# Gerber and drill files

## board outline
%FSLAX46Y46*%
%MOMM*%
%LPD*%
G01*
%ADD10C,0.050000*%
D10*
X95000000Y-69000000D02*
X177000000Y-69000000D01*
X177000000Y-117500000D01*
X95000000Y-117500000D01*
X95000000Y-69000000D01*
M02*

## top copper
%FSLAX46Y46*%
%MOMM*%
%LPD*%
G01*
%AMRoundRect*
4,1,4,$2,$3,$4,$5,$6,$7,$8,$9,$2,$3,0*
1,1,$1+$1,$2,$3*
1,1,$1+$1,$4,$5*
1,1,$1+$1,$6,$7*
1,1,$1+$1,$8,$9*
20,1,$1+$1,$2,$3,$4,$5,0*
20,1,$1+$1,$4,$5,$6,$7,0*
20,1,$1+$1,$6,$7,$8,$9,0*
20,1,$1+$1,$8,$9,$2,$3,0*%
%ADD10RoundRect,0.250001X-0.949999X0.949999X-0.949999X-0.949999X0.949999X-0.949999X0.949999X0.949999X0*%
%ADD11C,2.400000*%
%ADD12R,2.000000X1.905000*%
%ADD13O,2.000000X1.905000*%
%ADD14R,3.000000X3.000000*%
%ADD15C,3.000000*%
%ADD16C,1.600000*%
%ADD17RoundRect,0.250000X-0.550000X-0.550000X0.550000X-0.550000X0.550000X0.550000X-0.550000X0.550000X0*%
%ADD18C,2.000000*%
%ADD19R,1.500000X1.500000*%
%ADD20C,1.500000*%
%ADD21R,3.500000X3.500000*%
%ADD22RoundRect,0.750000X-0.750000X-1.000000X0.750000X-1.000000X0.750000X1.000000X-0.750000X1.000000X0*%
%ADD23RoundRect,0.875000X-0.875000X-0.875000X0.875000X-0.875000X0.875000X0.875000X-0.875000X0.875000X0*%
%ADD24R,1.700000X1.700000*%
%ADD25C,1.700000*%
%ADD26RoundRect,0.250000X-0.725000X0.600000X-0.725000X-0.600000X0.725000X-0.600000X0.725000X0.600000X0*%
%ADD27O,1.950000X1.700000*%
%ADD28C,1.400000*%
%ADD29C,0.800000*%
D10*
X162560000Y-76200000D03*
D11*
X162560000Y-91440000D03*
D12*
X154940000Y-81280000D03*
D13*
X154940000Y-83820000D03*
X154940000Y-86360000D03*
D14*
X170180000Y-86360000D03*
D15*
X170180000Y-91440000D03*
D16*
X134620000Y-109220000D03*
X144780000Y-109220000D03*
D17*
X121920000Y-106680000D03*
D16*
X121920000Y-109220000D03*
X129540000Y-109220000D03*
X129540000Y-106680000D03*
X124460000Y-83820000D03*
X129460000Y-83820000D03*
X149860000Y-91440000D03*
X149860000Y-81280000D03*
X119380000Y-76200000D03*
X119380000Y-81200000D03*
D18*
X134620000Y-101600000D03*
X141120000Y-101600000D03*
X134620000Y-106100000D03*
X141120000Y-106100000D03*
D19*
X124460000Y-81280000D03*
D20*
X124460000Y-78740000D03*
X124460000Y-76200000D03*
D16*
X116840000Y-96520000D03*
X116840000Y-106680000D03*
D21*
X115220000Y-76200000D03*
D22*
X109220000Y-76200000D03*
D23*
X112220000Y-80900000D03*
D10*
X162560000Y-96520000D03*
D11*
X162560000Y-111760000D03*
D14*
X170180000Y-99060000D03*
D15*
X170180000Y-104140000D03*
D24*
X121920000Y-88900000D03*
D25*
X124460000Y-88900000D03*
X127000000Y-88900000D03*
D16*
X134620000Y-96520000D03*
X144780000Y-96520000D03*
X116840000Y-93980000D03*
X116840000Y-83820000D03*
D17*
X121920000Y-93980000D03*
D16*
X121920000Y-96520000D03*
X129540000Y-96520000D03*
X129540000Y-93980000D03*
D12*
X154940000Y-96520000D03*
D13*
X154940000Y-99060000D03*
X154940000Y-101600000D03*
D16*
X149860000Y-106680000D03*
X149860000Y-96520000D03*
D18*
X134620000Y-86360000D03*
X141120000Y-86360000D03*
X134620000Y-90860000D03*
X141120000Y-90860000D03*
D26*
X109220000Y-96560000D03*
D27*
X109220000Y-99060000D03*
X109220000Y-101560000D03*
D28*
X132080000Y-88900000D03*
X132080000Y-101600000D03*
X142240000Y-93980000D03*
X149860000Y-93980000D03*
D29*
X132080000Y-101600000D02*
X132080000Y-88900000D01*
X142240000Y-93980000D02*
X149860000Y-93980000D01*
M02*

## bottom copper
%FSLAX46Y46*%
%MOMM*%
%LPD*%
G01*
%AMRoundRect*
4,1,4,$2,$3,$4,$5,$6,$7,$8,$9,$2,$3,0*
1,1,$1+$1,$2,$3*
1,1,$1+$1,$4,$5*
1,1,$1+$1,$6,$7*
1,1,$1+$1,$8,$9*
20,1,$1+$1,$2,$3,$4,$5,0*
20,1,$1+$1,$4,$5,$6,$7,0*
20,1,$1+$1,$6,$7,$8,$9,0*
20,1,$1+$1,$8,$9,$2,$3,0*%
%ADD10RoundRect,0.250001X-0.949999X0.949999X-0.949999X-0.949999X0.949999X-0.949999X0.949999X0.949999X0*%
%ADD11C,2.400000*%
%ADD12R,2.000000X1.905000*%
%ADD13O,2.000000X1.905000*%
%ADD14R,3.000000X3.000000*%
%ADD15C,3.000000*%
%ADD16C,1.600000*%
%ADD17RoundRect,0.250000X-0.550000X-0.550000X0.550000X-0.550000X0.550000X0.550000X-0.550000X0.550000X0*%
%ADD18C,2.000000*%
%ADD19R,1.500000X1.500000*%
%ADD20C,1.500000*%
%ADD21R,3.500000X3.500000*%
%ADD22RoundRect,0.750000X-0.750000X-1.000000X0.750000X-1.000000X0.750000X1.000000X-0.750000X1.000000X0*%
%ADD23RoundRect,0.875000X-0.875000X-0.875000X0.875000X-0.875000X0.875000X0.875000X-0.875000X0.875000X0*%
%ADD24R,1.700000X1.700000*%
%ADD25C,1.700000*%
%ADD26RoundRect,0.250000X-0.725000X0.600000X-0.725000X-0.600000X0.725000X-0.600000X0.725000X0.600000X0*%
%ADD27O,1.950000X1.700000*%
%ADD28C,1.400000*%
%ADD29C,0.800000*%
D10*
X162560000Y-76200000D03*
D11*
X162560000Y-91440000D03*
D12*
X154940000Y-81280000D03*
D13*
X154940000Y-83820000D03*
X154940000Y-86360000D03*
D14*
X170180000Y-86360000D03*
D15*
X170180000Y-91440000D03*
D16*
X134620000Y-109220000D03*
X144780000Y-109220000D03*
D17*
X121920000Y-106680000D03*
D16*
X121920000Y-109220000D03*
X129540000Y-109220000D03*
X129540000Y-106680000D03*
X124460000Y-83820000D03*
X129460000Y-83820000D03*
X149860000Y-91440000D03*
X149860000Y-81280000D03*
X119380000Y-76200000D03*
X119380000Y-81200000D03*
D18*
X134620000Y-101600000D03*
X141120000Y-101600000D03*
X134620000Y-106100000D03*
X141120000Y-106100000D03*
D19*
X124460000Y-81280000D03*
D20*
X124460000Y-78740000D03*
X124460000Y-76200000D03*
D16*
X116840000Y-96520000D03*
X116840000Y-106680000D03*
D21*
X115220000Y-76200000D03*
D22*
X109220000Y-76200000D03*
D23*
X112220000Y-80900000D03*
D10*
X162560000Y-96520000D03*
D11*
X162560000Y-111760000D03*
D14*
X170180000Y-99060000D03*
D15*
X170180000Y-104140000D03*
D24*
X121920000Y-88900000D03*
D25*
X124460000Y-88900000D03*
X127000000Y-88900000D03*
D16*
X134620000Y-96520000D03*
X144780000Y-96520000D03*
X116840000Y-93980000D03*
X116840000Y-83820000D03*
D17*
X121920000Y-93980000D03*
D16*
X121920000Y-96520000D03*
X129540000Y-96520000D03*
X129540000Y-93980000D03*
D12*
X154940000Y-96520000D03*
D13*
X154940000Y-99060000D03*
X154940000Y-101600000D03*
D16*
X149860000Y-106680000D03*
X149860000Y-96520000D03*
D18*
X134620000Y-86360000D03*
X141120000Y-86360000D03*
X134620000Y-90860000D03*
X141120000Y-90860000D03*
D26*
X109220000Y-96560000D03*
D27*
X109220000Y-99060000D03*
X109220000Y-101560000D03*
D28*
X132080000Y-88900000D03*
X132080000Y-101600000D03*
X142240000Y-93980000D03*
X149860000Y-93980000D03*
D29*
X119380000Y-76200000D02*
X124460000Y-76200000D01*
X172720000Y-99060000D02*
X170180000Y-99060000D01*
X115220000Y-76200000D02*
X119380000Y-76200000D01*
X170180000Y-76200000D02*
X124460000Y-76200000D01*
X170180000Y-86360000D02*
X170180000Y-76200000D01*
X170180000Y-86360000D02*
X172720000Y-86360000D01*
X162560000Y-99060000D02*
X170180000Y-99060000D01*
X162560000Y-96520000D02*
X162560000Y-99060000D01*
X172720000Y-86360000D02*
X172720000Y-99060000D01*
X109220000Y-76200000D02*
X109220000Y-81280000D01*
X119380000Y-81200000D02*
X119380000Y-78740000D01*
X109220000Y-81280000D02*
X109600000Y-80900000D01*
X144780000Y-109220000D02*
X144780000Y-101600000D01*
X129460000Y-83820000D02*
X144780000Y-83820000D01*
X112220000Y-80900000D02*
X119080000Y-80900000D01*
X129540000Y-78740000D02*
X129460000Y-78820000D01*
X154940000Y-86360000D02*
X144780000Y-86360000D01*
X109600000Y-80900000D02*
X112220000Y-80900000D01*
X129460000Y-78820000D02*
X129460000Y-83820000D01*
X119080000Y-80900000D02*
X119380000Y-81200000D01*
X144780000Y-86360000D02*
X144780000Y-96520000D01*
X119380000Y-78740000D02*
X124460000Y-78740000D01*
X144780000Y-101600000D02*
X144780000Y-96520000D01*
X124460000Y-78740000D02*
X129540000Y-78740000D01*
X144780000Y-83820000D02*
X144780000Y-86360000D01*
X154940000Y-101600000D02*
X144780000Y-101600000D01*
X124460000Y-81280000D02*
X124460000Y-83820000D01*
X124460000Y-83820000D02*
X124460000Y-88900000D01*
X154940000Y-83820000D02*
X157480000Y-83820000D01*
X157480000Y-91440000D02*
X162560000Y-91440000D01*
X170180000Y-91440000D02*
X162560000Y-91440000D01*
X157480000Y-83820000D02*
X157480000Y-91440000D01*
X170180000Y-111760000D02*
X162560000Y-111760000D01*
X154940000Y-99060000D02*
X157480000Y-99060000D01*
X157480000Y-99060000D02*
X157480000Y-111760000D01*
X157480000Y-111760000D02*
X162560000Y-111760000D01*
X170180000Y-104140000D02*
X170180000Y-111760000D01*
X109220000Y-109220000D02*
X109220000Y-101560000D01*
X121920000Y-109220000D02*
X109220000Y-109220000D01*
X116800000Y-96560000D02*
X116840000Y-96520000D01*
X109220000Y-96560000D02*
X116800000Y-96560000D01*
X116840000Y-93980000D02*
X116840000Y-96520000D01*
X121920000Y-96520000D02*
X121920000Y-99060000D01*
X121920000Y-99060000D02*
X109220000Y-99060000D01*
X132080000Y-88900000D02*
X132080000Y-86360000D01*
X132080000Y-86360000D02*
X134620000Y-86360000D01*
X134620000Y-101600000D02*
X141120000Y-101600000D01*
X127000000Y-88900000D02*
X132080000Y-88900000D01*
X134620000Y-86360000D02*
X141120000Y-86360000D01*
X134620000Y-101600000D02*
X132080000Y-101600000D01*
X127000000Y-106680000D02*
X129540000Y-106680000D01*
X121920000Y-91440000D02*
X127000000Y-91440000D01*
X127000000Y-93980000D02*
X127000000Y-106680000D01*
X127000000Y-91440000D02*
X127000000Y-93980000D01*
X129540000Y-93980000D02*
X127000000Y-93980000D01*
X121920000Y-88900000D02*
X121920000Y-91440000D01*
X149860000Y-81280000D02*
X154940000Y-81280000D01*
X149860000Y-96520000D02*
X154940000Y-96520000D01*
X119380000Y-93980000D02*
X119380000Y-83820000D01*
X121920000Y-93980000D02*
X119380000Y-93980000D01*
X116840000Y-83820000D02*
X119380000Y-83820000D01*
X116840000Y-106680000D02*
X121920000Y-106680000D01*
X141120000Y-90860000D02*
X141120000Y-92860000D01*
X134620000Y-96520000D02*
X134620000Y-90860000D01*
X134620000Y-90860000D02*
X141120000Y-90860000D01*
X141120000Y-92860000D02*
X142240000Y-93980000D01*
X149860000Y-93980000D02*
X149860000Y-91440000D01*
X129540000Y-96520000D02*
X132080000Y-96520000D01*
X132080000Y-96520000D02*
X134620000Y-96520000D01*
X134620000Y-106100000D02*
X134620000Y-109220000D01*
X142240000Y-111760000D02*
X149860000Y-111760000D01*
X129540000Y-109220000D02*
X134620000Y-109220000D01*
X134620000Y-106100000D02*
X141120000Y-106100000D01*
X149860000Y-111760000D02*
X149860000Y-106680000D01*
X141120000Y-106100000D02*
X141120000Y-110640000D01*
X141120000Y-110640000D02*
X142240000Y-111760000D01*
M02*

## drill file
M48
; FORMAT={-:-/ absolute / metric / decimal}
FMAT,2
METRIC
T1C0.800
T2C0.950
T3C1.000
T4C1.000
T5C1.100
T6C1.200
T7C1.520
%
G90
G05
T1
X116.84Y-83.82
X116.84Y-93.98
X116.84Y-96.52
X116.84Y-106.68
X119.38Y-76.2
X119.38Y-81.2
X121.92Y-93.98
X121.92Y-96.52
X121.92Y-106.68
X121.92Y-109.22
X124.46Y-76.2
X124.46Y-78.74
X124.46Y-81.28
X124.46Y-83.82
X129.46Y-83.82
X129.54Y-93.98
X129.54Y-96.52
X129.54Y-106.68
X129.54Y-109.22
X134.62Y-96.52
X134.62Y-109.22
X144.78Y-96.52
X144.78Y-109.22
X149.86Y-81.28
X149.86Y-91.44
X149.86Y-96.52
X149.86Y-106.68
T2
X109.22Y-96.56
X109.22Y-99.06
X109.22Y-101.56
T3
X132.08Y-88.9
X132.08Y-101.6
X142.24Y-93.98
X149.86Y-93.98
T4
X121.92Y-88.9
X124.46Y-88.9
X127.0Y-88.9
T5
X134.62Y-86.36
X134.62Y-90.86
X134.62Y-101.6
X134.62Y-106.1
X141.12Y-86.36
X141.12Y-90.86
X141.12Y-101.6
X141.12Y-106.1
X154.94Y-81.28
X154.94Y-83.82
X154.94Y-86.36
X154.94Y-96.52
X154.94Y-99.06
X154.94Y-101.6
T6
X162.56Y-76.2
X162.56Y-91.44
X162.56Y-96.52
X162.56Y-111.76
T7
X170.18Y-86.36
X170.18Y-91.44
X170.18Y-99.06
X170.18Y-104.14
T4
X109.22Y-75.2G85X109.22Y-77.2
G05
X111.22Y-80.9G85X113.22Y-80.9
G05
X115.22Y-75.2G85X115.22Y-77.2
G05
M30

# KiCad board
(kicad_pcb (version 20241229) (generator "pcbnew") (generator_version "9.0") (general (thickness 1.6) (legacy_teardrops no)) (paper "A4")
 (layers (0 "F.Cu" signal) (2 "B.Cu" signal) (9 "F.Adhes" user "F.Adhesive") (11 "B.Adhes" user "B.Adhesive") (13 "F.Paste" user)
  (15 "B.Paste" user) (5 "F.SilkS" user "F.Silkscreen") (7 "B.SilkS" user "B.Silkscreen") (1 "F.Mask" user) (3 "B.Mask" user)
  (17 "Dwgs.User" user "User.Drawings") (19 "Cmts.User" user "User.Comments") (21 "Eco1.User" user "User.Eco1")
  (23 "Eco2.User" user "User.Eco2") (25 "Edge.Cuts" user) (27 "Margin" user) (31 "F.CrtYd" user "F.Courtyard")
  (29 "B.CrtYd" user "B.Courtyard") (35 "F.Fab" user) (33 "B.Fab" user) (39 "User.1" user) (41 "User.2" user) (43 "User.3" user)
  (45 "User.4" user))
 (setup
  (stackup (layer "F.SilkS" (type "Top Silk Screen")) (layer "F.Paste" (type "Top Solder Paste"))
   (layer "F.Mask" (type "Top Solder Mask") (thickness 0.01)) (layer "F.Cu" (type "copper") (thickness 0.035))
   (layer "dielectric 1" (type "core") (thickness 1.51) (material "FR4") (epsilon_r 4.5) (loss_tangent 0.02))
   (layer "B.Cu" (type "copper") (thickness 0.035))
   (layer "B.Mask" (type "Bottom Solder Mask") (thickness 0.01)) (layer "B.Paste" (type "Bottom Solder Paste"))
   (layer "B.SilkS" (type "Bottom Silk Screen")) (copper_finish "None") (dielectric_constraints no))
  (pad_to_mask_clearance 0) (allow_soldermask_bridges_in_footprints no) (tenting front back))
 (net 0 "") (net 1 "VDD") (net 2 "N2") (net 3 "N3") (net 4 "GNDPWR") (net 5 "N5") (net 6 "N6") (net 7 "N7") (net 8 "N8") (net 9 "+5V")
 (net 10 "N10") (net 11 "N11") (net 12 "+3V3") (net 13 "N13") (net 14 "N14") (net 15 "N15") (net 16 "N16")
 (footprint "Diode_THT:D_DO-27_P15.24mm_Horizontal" (layer "F.Cu") (at 162.56 76.2 -90)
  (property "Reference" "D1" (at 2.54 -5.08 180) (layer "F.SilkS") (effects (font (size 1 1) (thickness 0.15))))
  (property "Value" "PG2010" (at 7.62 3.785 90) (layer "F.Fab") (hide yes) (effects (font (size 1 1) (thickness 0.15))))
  (pad "1" thru_hole roundrect (at 0 0 270) (size 2.4 2.4) (drill 1.2) (layers "*.Cu" "*.Mask") (remove_unused_layers no)
   (roundrect_rratio 0.104167) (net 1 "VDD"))
  (pad "2" thru_hole circle (at 15.24 0 270) (size 2.4 2.4) (drill 1.2) (layers "*.Cu" "*.Mask") (remove_unused_layers no) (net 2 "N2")))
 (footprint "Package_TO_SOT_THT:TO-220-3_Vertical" (layer "F.Cu") (at 154.94 81.28 -90)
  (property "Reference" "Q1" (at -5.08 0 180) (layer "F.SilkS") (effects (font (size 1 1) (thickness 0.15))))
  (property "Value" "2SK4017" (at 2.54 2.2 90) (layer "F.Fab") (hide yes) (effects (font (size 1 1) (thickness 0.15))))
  (pad "1" thru_hole rect (at 0 0 270) (size 1.905 2) (drill 1.1) (layers "*.Cu" "*.Mask") (remove_unused_layers no) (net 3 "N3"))
  (pad "2" thru_hole oval (at 2.54 0 270) (size 1.905 2) (drill 1.1) (layers "*.Cu" "*.Mask") (remove_unused_layers no) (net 2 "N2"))
  (pad "3" thru_hole oval (at 5.08 0 270) (size 1.905 2) (drill 1.1) (layers "*.Cu" "*.Mask") (remove_unused_layers no) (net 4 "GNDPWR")))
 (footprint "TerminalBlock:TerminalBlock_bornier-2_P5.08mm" (layer "F.Cu") (at 170.18 86.36 -90)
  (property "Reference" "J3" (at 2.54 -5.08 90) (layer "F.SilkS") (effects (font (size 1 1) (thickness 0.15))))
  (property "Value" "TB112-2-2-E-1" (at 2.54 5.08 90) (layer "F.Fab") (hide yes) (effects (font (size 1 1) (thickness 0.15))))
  (pad "1" thru_hole rect (at 0 0 270) (size 3 3) (drill 1.52) (layers "*.Cu" "*.Mask") (remove_unused_layers no) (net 1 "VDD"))
  (pad "2" thru_hole circle (at 5.08 0 270) (size 3 3) (drill 1.52) (layers "*.Cu" "*.Mask") (remove_unused_layers no) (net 2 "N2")))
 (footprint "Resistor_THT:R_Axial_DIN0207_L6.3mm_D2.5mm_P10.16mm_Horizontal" (layer "F.Cu") (at 134.62 109.22)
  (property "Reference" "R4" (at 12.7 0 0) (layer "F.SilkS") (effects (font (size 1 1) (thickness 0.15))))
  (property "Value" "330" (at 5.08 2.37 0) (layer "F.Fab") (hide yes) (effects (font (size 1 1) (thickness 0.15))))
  (pad "1" thru_hole circle (at 0 0) (size 1.6 1.6) (drill 0.8) (layers "*.Cu" "*.Mask") (remove_unused_layers no) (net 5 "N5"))
  (pad "2" thru_hole circle (at 10.16 0) (size 1.6 1.6) (drill 0.8) (layers "*.Cu" "*.Mask") (remove_unused_layers no) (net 4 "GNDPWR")))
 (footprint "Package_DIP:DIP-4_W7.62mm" (layer "F.Cu") (at 121.92 106.68)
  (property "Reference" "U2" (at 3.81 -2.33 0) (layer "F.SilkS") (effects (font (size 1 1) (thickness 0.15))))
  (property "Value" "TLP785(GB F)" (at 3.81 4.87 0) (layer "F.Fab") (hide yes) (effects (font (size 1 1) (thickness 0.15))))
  (pad "1" thru_hole roundrect (at 0 0) (size 1.6 1.6) (drill 0.8) (layers "*.Cu" "*.Mask") (remove_unused_layers no)
   (roundrect_rratio 0.15625) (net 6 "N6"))
  (pad "2" thru_hole circle (at 0 2.54) (size 1.6 1.6) (drill 0.8) (layers "*.Cu" "*.Mask") (remove_unused_layers no) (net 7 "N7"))
  (pad "3" thru_hole circle (at 7.62 2.54) (size 1.6 1.6) (drill 0.8) (layers "*.Cu" "*.Mask") (remove_unused_layers no) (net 5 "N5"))
  (pad "4" thru_hole circle (at 7.62 0) (size 1.6 1.6) (drill 0.8) (layers "*.Cu" "*.Mask") (remove_unused_layers no) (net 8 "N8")))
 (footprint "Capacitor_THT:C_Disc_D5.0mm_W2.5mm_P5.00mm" (layer "F.Cu") (at 124.46 83.82)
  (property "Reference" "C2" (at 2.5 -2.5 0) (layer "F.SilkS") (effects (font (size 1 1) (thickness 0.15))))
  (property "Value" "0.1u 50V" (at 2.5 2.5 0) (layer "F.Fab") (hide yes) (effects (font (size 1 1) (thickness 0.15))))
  (pad "1" thru_hole circle (at 0 0) (size 1.6 1.6) (drill 0.8) (layers "*.Cu" "*.Mask") (remove_unused_layers no) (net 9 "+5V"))
  (pad "2" thru_hole circle (at 5 0) (size 1.6 1.6) (drill 0.8) (layers "*.Cu" "*.Mask") (remove_unused_layers no) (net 4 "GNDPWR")))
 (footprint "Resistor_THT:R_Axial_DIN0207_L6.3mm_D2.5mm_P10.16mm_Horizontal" (layer "F.Cu") (at 149.86 91.44 90)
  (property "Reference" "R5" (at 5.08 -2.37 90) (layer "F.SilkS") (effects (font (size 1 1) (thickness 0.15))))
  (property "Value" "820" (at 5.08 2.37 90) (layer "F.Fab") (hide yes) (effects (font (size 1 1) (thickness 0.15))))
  (pad "1" thru_hole circle (at 0 0 90) (size 1.6 1.6) (drill 0.8) (layers "*.Cu" "*.Mask") (remove_unused_layers no) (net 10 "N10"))
  (pad "2" thru_hole circle (at 10.16 0 90) (size 1.6 1.6) (drill 0.8) (layers "*.Cu" "*.Mask") (remove_unused_layers no) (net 3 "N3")))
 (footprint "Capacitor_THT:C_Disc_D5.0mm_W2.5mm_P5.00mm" (layer "F.Cu") (at 119.38 76.2 -90)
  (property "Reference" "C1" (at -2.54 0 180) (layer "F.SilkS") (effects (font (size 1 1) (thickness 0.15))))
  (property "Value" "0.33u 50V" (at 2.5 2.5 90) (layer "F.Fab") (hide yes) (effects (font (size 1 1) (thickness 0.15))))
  (pad "1" thru_hole circle (at 0 0 270) (size 1.6 1.6) (drill 0.8) (layers "*.Cu" "*.Mask") (remove_unused_layers no) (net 1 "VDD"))
  (pad "2" thru_hole circle (at 5 0 270) (size 1.6 1.6) (drill 0.8) (layers "*.Cu" "*.Mask") (remove_unused_layers no) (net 4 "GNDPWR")))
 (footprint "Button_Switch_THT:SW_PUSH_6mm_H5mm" (layer "F.Cu") (at 134.62 101.6)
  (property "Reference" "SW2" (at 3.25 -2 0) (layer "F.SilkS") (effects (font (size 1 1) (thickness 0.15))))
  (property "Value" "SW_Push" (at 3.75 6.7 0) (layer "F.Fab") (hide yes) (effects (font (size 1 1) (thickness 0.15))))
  (pad "1" thru_hole circle (at 0 0 90) (size 2 2) (drill 1.1) (layers "*.Cu" "*.Mask") (remove_unused_layers no) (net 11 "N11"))
  (pad "1" thru_hole circle (at 6.5 0 90) (size 2 2) (drill 1.1) (layers "*.Cu" "*.Mask") (remove_unused_layers no) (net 11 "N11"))
  (pad "2" thru_hole circle (at 0 4.5 90) (size 2 2) (drill 1.1) (layers "*.Cu" "*.Mask") (remove_unused_layers no) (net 5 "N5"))
  (pad "2" thru_hole circle (at 6.5 4.5 90) (size 2 2) (drill 1.1) (layers "*.Cu" "*.Mask") (remove_unused_layers no) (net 5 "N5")))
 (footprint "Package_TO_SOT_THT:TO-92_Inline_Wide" (layer "F.Cu") (at 124.46 81.28 90)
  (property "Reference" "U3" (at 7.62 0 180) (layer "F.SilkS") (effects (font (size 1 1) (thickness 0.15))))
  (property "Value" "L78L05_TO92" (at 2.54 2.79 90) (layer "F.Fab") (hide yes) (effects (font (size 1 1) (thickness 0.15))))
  (pad "1" thru_hole rect (at 0 0 90) (size 1.5 1.5) (drill 0.8) (layers "*.Cu" "*.Mask") (remove_unused_layers no) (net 9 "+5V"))
  (pad "2" thru_hole circle (at 2.54 0 90) (size 1.5 1.5) (drill 0.8) (layers "*.Cu" "*.Mask") (remove_unused_layers no) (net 4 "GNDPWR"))
  (pad "3" thru_hole circle (at 5.08 0 90) (size 1.5 1.5) (drill 0.8) (layers "*.Cu" "*.Mask") (remove_unused_layers no) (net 1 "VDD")))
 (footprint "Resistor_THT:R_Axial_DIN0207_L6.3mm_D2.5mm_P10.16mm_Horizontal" (layer "F.Cu") (at 116.84 96.52 -90)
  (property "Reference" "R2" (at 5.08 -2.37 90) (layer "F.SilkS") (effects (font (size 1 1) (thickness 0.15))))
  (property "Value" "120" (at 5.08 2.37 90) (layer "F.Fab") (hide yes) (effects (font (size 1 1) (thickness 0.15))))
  (pad "1" thru_hole circle (at 0 0 270) (size 1.6 1.6) (drill 0.8) (layers "*.Cu" "*.Mask") (remove_unused_layers no) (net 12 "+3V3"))
  (pad "2" thru_hole circle (at 10.16 0 270) (size 1.6 1.6) (drill 0.8) (layers "*.Cu" "*.Mask") (remove_unused_layers no) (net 6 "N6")))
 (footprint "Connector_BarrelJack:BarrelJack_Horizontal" (layer "F.Cu") (at 115.22 76.2)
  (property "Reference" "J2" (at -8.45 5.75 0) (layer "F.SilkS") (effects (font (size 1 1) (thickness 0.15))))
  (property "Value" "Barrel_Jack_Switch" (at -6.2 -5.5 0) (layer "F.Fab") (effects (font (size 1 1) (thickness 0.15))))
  (pad "1" thru_hole rect (at 0 0) (size 3.5 3.5) (drill oval 1 3) (layers "*.Cu" "*.Mask") (remove_unused_layers no) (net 1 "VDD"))
  (pad "2" thru_hole roundrect (at -6 0) (size 3 3.5) (drill oval 1 3) (layers "*.Cu" "*.Mask") (remove_unused_layers no)
   (roundrect_rratio 0.25) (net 4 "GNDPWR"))
  (pad "3" thru_hole roundrect (at -3 4.7) (size 3.5 3.5) (drill oval 3 1) (layers "*.Cu" "*.Mask") (remove_unused_layers no)
   (roundrect_rratio 0.25) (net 4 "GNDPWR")))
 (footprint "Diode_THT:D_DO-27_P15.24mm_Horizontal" (layer "F.Cu") (at 162.56 96.52 -90)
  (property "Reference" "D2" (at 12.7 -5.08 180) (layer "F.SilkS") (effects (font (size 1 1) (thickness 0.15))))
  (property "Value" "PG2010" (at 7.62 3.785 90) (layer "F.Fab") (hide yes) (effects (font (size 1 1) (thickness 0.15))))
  (pad "1" thru_hole roundrect (at 0 0 270) (size 2.4 2.4) (drill 1.2) (layers "*.Cu" "*.Mask") (remove_unused_layers no)
   (roundrect_rratio 0.104167) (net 1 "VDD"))
  (pad "2" thru_hole circle (at 15.24 0 270) (size 2.4 2.4) (drill 1.2) (layers "*.Cu" "*.Mask") (remove_unused_layers no) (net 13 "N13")))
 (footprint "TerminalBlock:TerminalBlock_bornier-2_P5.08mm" (layer "F.Cu") (at 170.18 99.06 -90)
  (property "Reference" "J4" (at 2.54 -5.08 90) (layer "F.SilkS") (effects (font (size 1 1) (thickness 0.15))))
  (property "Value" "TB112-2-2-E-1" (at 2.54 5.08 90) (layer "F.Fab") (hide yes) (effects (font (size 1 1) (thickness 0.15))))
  (pad "1" thru_hole rect (at 0 0 270) (size 3 3) (drill 1.52) (layers "*.Cu" "*.Mask") (remove_unused_layers no) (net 1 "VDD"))
  (pad "2" thru_hole circle (at 5.08 0 270) (size 3 3) (drill 1.52) (layers "*.Cu" "*.Mask") (remove_unused_layers no) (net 13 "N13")))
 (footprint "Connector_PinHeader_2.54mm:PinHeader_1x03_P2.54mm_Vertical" (layer "F.Cu") (at 121.92 88.9 90)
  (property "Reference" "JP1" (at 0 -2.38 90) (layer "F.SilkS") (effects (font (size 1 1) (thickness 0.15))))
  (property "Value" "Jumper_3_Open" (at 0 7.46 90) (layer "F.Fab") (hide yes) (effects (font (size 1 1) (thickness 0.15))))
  (pad "1" thru_hole rect (at 0 0 90) (size 1.7 1.7) (drill 1) (layers "*.Cu" "*.Mask") (remove_unused_layers no) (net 8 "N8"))
  (pad "2" thru_hole circle (at 0 2.54 90) (size 1.7 1.7) (drill 1) (layers "*.Cu" "*.Mask") (remove_unused_layers no) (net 9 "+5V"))
  (pad "3" thru_hole circle (at 0 5.08 90) (size 1.7 1.7) (drill 1) (layers "*.Cu" "*.Mask") (remove_unused_layers no) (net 11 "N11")))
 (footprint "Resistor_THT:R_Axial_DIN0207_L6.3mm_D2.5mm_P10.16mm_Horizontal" (layer "F.Cu") (at 134.62 96.52)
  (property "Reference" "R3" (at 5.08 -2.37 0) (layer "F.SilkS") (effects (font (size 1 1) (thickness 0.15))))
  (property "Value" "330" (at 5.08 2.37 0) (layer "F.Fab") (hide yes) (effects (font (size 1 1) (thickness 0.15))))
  (pad "1" thru_hole circle (at 0 0) (size 1.6 1.6) (drill 0.8) (layers "*.Cu" "*.Mask") (remove_unused_layers no) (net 10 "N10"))
  (pad "2" thru_hole circle (at 10.16 0) (size 1.6 1.6) (drill 0.8) (layers "*.Cu" "*.Mask") (remove_unused_layers no) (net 4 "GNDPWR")))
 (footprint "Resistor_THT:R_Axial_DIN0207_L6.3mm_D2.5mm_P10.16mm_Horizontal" (layer "F.Cu") (at 116.84 93.98 90)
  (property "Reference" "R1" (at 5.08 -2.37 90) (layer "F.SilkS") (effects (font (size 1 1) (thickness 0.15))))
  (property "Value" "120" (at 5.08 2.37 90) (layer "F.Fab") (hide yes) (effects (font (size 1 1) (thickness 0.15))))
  (pad "1" thru_hole circle (at 0 0 90) (size 1.6 1.6) (drill 0.8) (layers "*.Cu" "*.Mask") (remove_unused_layers no) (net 12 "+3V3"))
  (pad "2" thru_hole circle (at 10.16 0 90) (size 1.6 1.6) (drill 0.8) (layers "*.Cu" "*.Mask") (remove_unused_layers no) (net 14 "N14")))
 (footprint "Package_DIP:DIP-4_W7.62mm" (layer "F.Cu") (at 121.92 93.98)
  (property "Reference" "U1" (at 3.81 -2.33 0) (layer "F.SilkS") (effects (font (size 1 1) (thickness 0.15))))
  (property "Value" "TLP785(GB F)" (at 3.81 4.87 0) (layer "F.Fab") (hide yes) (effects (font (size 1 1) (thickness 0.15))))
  (pad "1" thru_hole roundrect (at 0 0) (size 1.6 1.6) (drill 0.8) (layers "*.Cu" "*.Mask") (remove_unused_layers no)
   (roundrect_rratio 0.15625) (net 14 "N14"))
  (pad "2" thru_hole circle (at 0 2.54) (size 1.6 1.6) (drill 0.8) (layers "*.Cu" "*.Mask") (remove_unused_layers no) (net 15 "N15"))
  (pad "3" thru_hole circle (at 7.62 2.54) (size 1.6 1.6) (drill 0.8) (layers "*.Cu" "*.Mask") (remove_unused_layers no) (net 10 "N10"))
  (pad "4" thru_hole circle (at 7.62 0) (size 1.6 1.6) (drill 0.8) (layers "*.Cu" "*.Mask") (remove_unused_layers no) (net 8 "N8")))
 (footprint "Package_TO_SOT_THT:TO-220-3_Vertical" (layer "F.Cu") (at 154.94 96.52 -90)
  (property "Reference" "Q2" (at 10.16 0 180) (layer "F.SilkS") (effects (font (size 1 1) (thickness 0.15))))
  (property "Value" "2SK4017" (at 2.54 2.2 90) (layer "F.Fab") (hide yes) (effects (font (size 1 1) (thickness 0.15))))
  (pad "1" thru_hole rect (at 0 0 270) (size 1.905 2) (drill 1.1) (layers "*.Cu" "*.Mask") (remove_unused_layers no) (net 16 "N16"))
  (pad "2" thru_hole oval (at 2.54 0 270) (size 1.905 2) (drill 1.1) (layers "*.Cu" "*.Mask") (remove_unused_layers no) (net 13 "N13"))
  (pad "3" thru_hole oval (at 5.08 0 270) (size 1.905 2) (drill 1.1) (layers "*.Cu" "*.Mask") (remove_unused_layers no) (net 4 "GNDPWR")))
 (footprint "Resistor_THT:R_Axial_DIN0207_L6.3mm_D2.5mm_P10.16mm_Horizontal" (layer "F.Cu") (at 149.86 106.68 90)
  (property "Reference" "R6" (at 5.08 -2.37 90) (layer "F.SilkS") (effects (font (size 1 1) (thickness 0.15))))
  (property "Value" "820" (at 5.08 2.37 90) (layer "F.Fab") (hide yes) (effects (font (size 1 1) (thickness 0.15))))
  (pad "1" thru_hole circle (at 0 0 90) (size 1.6 1.6) (drill 0.8) (layers "*.Cu" "*.Mask") (remove_unused_layers no) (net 5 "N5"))
  (pad "2" thru_hole circle (at 10.16 0 90) (size 1.6 1.6) (drill 0.8) (layers "*.Cu" "*.Mask") (remove_unused_layers no) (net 16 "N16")))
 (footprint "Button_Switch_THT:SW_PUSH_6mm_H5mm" (layer "F.Cu") (at 134.62 86.36)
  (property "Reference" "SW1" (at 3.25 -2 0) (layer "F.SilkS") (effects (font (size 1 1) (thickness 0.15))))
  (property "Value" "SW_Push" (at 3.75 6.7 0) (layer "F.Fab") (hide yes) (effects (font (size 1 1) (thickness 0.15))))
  (pad "1" thru_hole circle (at 0 0 90) (size 2 2) (drill 1.1) (layers "*.Cu" "*.Mask") (remove_unused_layers no) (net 11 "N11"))
  (pad "1" thru_hole circle (at 6.5 0 90) (size 2 2) (drill 1.1) (layers "*.Cu" "*.Mask") (remove_unused_layers no) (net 11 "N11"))
  (pad "2" thru_hole circle (at 0 4.5 90) (size 2 2) (drill 1.1) (layers "*.Cu" "*.Mask") (remove_unused_layers no) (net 10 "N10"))
  (pad "2" thru_hole circle (at 6.5 4.5 90) (size 2 2) (drill 1.1) (layers "*.Cu" "*.Mask") (remove_unused_layers no) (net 10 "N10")))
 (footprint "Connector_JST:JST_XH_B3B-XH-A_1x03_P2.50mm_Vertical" (layer "F.Cu") (at 109.22 96.56 -90)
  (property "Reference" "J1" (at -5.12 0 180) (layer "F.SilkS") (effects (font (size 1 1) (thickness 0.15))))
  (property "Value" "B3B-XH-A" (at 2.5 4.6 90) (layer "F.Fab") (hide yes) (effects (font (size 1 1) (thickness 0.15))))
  (pad "1" thru_hole roundrect (at 0 0 270) (size 1.7 1.95) (drill 0.95) (layers "*.Cu" "*.Mask") (remove_unused_layers no)
   (roundrect_rratio 0.147059) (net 12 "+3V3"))
  (pad "2" thru_hole oval (at 2.5 0 270) (size 1.7 1.95) (drill 0.95) (layers "*.Cu" "*.Mask") (remove_unused_layers no) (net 15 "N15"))
  (pad "3" thru_hole oval (at 5 0 270) (size 1.7 1.95) (drill 0.95) (layers "*.Cu" "*.Mask") (remove_unused_layers no) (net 7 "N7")))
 (gr_rect (start 95 69) (end 177 117.5) (stroke (width 0.05) (type default)) (fill no) (layer "Edge.Cuts"))
 (segment (start 119.38 76.2) (end 124.46 76.2) (width 0.8) (layer "B.Cu") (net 1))
 (segment (start 172.72 99.06) (end 170.18 99.06) (width 0.8) (layer "B.Cu") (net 1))
 (segment (start 115.22 76.2) (end 119.38 76.2) (width 0.8) (layer "B.Cu") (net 1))
 (segment (start 170.18 76.2) (end 124.46 76.2) (width 0.8) (layer "B.Cu") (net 1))
 (segment (start 170.18 86.36) (end 170.18 76.2) (width 0.8) (layer "B.Cu") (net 1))
 (segment (start 170.18 86.36) (end 172.72 86.36) (width 0.8) (layer "B.Cu") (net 1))
 (segment (start 162.56 99.06) (end 170.18 99.06) (width 0.8) (layer "B.Cu") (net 1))
 (segment (start 162.56 96.52) (end 162.56 99.06) (width 0.8) (layer "B.Cu") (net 1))
 (segment (start 172.72 86.36) (end 172.72 99.06) (width 0.8) (layer "B.Cu") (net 1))
 (segment (start 109.22 76.2) (end 109.22 81.28) (width 0.8) (layer "B.Cu") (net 4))
 (segment (start 119.38 81.2) (end 119.38 78.74) (width 0.8) (layer "B.Cu") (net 4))
 (segment (start 109.22 81.28) (end 109.6 80.9) (width 0.8) (layer "B.Cu") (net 4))
 (segment (start 144.78 109.22) (end 144.78 101.6) (width 0.8) (layer "B.Cu") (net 4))
 (segment (start 129.46 83.82) (end 144.78 83.82) (width 0.8) (layer "B.Cu") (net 4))
 (segment (start 112.22 80.9) (end 119.08 80.9) (width 0.8) (layer "B.Cu") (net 4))
 (segment (start 129.54 78.74) (end 129.46 78.82) (width 0.8) (layer "B.Cu") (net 4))
 (segment (start 154.94 86.36) (end 144.78 86.36) (width 0.8) (layer "B.Cu") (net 4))
 (segment (start 109.6 80.9) (end 112.22 80.9) (width 0.8) (layer "B.Cu") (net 4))
 (segment (start 129.46 78.82) (end 129.46 83.82) (width 0.8) (layer "B.Cu") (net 4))
 (segment (start 119.08 80.9) (end 119.38 81.2) (width 0.8) (layer "B.Cu") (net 4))
 (segment (start 144.78 86.36) (end 144.78 96.52) (width 0.8) (layer "B.Cu") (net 4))
 (segment (start 119.38 78.74) (end 124.46 78.74) (width 0.8) (layer "B.Cu") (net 4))
 (segment (start 144.78 101.6) (end 144.78 96.52) (width 0.8) (layer "B.Cu") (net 4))
 (segment (start 124.46 78.74) (end 129.54 78.74) (width 0.8) (layer "B.Cu") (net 4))
 (segment (start 144.78 83.82) (end 144.78 86.36) (width 0.8) (layer "B.Cu") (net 4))
 (segment (start 154.94 101.6) (end 144.78 101.6) (width 0.8) (layer "B.Cu") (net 4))
 (segment (start 124.46 81.28) (end 124.46 83.82) (width 0.8) (layer "B.Cu") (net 9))
 (segment (start 124.46 83.82) (end 124.46 88.9) (width 0.8) (layer "B.Cu") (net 9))
 (segment (start 154.94 83.82) (end 157.48 83.82) (width 0.8) (layer "B.Cu") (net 2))
 (segment (start 157.48 91.44) (end 162.56 91.44) (width 0.8) (layer "B.Cu") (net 2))
 (segment (start 170.18 91.44) (end 162.56 91.44) (width 0.8) (layer "B.Cu") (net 2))
 (segment (start 157.48 83.82) (end 157.48 91.44) (width 0.8) (layer "B.Cu") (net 2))
 (segment (start 170.18 111.76) (end 162.56 111.76) (width 0.8) (layer "B.Cu") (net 13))
 (segment (start 154.94 99.06) (end 157.48 99.06) (width 0.8) (layer "B.Cu") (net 13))
 (segment (start 157.48 99.06) (end 157.48 111.76) (width 0.8) (layer "B.Cu") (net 13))
 (segment (start 157.48 111.76) (end 162.56 111.76) (width 0.8) (layer "B.Cu") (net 13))
 (segment (start 170.18 104.14) (end 170.18 111.76) (width 0.8) (layer "B.Cu") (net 13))
 (segment (start 109.22 109.22) (end 109.22 101.56) (width 0.8) (layer "B.Cu") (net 7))
 (segment (start 121.92 109.22) (end 109.22 109.22) (width 0.8) (layer "B.Cu") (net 7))
 (segment (start 116.8 96.56) (end 116.84 96.52) (width 0.8) (layer "B.Cu") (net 12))
 (segment (start 109.22 96.56) (end 116.8 96.56) (width 0.8) (layer "B.Cu") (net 12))
 (segment (start 116.84 93.98) (end 116.84 96.52) (width 0.8) (layer "B.Cu") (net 12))
 (segment (start 121.92 96.52) (end 121.92 99.06) (width 0.8) (layer "B.Cu") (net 15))
 (segment (start 121.92 99.06) (end 109.22 99.06) (width 0.8) (layer "B.Cu") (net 15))
 (segment (start 132.08 101.6) (end 132.08 88.9) (width 0.8) (layer "F.Cu") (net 11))
 (via (at 132.08 88.9) (size 1.4) (drill 1) (layers "F.Cu" "B.Cu") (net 11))
 (via (at 132.08 101.6) (size 1.4) (drill 1) (layers "F.Cu" "B.Cu") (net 11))
 (segment (start 132.08 88.9) (end 132.08 86.36) (width 0.8) (layer "B.Cu") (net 11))
 (segment (start 132.08 86.36) (end 134.62 86.36) (width 0.8) (layer "B.Cu") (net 11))
 (segment (start 134.62 101.6) (end 141.12 101.6) (width 0.8) (layer "B.Cu") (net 11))
 (segment (start 127 88.9) (end 132.08 88.9) (width 0.8) (layer "B.Cu") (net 11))
 (segment (start 134.62 86.36) (end 141.12 86.36) (width 0.8) (layer "B.Cu") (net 11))
 (segment (start 134.62 101.6) (end 132.08 101.6) (width 0.8) (layer "B.Cu") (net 11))
 (segment (start 127 106.68) (end 129.54 106.68) (width 0.8) (layer "B.Cu") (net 8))
 (segment (start 121.92 91.44) (end 127 91.44) (width 0.8) (layer "B.Cu") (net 8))
 (segment (start 127 93.98) (end 127 106.68) (width 0.8) (layer "B.Cu") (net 8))
 (segment (start 127 91.44) (end 127 93.98) (width 0.8) (layer "B.Cu") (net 8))
 (segment (start 129.54 93.98) (end 127 93.98) (width 0.8) (layer "B.Cu") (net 8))
 (segment (start 121.92 88.9) (end 121.92 91.44) (width 0.8) (layer "B.Cu") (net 8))
 (segment (start 149.86 81.28) (end 154.94 81.28) (width 0.8) (layer "B.Cu") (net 3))
 (segment (start 149.86 96.52) (end 154.94 96.52) (width 0.8) (layer "B.Cu") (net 16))
 (segment (start 119.38 93.98) (end 119.38 83.82) (width 0.8) (layer "B.Cu") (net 14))
 (segment (start 121.92 93.98) (end 119.38 93.98) (width 0.8) (layer "B.Cu") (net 14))
 (segment (start 116.84 83.82) (end 119.38 83.82) (width 0.8) (layer "B.Cu") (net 14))
 (segment (start 116.84 106.68) (end 121.92 106.68) (width 0.8) (layer "B.Cu") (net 6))
 (segment (start 142.24 93.98) (end 149.86 93.98) (width 0.8) (layer "F.Cu") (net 10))
 (via (at 142.24 93.98) (size 1.4) (drill 1) (layers "F.Cu" "B.Cu") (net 10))
 (via (at 149.86 93.98) (size 1.4) (drill 1) (layers "F.Cu" "B.Cu") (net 10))
 (segment (start 141.12 90.86) (end 141.12 92.86) (width 0.8) (layer "B.Cu") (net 10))
 (segment (start 134.62 96.52) (end 134.62 90.86) (width 0.8) (layer "B.Cu") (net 10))
 (segment (start 134.62 90.86) (end 141.12 90.86) (width 0.8) (layer "B.Cu") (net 10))
 (segment (start 141.12 92.86) (end 142.24 93.98) (width 0.8) (layer "B.Cu") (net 10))
 (segment (start 149.86 93.98) (end 149.86 91.44) (width 0.8) (layer "B.Cu") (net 10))
 (segment (start 129.54 96.52) (end 132.08 96.52) (width 0.8) (layer "B.Cu") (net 10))
 (segment (start 132.08 96.52) (end 134.62 96.52) (width 0.8) (layer "B.Cu") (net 10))
 (segment (start 134.62 106.1) (end 134.62 109.22) (width 0.8) (layer "B.Cu") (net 5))
 (segment (start 142.24 111.76) (end 149.86 111.76) (width 0.8) (layer "B.Cu") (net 5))
 (segment (start 129.54 109.22) (end 134.62 109.22) (width 0.8) (layer "B.Cu") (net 5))
 (segment (start 134.62 106.1) (end 141.12 106.1) (width 0.8) (layer "B.Cu") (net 5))
 (segment (start 149.86 111.76) (end 149.86 106.68) (width 0.8) (layer "B.Cu") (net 5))
 (segment (start 141.12 106.1) (end 141.12 110.64) (width 0.8) (layer "B.Cu") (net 5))
 (segment (start 141.12 110.64) (end 142.24 111.76) (width 0.8) (layer "B.Cu") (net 5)))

